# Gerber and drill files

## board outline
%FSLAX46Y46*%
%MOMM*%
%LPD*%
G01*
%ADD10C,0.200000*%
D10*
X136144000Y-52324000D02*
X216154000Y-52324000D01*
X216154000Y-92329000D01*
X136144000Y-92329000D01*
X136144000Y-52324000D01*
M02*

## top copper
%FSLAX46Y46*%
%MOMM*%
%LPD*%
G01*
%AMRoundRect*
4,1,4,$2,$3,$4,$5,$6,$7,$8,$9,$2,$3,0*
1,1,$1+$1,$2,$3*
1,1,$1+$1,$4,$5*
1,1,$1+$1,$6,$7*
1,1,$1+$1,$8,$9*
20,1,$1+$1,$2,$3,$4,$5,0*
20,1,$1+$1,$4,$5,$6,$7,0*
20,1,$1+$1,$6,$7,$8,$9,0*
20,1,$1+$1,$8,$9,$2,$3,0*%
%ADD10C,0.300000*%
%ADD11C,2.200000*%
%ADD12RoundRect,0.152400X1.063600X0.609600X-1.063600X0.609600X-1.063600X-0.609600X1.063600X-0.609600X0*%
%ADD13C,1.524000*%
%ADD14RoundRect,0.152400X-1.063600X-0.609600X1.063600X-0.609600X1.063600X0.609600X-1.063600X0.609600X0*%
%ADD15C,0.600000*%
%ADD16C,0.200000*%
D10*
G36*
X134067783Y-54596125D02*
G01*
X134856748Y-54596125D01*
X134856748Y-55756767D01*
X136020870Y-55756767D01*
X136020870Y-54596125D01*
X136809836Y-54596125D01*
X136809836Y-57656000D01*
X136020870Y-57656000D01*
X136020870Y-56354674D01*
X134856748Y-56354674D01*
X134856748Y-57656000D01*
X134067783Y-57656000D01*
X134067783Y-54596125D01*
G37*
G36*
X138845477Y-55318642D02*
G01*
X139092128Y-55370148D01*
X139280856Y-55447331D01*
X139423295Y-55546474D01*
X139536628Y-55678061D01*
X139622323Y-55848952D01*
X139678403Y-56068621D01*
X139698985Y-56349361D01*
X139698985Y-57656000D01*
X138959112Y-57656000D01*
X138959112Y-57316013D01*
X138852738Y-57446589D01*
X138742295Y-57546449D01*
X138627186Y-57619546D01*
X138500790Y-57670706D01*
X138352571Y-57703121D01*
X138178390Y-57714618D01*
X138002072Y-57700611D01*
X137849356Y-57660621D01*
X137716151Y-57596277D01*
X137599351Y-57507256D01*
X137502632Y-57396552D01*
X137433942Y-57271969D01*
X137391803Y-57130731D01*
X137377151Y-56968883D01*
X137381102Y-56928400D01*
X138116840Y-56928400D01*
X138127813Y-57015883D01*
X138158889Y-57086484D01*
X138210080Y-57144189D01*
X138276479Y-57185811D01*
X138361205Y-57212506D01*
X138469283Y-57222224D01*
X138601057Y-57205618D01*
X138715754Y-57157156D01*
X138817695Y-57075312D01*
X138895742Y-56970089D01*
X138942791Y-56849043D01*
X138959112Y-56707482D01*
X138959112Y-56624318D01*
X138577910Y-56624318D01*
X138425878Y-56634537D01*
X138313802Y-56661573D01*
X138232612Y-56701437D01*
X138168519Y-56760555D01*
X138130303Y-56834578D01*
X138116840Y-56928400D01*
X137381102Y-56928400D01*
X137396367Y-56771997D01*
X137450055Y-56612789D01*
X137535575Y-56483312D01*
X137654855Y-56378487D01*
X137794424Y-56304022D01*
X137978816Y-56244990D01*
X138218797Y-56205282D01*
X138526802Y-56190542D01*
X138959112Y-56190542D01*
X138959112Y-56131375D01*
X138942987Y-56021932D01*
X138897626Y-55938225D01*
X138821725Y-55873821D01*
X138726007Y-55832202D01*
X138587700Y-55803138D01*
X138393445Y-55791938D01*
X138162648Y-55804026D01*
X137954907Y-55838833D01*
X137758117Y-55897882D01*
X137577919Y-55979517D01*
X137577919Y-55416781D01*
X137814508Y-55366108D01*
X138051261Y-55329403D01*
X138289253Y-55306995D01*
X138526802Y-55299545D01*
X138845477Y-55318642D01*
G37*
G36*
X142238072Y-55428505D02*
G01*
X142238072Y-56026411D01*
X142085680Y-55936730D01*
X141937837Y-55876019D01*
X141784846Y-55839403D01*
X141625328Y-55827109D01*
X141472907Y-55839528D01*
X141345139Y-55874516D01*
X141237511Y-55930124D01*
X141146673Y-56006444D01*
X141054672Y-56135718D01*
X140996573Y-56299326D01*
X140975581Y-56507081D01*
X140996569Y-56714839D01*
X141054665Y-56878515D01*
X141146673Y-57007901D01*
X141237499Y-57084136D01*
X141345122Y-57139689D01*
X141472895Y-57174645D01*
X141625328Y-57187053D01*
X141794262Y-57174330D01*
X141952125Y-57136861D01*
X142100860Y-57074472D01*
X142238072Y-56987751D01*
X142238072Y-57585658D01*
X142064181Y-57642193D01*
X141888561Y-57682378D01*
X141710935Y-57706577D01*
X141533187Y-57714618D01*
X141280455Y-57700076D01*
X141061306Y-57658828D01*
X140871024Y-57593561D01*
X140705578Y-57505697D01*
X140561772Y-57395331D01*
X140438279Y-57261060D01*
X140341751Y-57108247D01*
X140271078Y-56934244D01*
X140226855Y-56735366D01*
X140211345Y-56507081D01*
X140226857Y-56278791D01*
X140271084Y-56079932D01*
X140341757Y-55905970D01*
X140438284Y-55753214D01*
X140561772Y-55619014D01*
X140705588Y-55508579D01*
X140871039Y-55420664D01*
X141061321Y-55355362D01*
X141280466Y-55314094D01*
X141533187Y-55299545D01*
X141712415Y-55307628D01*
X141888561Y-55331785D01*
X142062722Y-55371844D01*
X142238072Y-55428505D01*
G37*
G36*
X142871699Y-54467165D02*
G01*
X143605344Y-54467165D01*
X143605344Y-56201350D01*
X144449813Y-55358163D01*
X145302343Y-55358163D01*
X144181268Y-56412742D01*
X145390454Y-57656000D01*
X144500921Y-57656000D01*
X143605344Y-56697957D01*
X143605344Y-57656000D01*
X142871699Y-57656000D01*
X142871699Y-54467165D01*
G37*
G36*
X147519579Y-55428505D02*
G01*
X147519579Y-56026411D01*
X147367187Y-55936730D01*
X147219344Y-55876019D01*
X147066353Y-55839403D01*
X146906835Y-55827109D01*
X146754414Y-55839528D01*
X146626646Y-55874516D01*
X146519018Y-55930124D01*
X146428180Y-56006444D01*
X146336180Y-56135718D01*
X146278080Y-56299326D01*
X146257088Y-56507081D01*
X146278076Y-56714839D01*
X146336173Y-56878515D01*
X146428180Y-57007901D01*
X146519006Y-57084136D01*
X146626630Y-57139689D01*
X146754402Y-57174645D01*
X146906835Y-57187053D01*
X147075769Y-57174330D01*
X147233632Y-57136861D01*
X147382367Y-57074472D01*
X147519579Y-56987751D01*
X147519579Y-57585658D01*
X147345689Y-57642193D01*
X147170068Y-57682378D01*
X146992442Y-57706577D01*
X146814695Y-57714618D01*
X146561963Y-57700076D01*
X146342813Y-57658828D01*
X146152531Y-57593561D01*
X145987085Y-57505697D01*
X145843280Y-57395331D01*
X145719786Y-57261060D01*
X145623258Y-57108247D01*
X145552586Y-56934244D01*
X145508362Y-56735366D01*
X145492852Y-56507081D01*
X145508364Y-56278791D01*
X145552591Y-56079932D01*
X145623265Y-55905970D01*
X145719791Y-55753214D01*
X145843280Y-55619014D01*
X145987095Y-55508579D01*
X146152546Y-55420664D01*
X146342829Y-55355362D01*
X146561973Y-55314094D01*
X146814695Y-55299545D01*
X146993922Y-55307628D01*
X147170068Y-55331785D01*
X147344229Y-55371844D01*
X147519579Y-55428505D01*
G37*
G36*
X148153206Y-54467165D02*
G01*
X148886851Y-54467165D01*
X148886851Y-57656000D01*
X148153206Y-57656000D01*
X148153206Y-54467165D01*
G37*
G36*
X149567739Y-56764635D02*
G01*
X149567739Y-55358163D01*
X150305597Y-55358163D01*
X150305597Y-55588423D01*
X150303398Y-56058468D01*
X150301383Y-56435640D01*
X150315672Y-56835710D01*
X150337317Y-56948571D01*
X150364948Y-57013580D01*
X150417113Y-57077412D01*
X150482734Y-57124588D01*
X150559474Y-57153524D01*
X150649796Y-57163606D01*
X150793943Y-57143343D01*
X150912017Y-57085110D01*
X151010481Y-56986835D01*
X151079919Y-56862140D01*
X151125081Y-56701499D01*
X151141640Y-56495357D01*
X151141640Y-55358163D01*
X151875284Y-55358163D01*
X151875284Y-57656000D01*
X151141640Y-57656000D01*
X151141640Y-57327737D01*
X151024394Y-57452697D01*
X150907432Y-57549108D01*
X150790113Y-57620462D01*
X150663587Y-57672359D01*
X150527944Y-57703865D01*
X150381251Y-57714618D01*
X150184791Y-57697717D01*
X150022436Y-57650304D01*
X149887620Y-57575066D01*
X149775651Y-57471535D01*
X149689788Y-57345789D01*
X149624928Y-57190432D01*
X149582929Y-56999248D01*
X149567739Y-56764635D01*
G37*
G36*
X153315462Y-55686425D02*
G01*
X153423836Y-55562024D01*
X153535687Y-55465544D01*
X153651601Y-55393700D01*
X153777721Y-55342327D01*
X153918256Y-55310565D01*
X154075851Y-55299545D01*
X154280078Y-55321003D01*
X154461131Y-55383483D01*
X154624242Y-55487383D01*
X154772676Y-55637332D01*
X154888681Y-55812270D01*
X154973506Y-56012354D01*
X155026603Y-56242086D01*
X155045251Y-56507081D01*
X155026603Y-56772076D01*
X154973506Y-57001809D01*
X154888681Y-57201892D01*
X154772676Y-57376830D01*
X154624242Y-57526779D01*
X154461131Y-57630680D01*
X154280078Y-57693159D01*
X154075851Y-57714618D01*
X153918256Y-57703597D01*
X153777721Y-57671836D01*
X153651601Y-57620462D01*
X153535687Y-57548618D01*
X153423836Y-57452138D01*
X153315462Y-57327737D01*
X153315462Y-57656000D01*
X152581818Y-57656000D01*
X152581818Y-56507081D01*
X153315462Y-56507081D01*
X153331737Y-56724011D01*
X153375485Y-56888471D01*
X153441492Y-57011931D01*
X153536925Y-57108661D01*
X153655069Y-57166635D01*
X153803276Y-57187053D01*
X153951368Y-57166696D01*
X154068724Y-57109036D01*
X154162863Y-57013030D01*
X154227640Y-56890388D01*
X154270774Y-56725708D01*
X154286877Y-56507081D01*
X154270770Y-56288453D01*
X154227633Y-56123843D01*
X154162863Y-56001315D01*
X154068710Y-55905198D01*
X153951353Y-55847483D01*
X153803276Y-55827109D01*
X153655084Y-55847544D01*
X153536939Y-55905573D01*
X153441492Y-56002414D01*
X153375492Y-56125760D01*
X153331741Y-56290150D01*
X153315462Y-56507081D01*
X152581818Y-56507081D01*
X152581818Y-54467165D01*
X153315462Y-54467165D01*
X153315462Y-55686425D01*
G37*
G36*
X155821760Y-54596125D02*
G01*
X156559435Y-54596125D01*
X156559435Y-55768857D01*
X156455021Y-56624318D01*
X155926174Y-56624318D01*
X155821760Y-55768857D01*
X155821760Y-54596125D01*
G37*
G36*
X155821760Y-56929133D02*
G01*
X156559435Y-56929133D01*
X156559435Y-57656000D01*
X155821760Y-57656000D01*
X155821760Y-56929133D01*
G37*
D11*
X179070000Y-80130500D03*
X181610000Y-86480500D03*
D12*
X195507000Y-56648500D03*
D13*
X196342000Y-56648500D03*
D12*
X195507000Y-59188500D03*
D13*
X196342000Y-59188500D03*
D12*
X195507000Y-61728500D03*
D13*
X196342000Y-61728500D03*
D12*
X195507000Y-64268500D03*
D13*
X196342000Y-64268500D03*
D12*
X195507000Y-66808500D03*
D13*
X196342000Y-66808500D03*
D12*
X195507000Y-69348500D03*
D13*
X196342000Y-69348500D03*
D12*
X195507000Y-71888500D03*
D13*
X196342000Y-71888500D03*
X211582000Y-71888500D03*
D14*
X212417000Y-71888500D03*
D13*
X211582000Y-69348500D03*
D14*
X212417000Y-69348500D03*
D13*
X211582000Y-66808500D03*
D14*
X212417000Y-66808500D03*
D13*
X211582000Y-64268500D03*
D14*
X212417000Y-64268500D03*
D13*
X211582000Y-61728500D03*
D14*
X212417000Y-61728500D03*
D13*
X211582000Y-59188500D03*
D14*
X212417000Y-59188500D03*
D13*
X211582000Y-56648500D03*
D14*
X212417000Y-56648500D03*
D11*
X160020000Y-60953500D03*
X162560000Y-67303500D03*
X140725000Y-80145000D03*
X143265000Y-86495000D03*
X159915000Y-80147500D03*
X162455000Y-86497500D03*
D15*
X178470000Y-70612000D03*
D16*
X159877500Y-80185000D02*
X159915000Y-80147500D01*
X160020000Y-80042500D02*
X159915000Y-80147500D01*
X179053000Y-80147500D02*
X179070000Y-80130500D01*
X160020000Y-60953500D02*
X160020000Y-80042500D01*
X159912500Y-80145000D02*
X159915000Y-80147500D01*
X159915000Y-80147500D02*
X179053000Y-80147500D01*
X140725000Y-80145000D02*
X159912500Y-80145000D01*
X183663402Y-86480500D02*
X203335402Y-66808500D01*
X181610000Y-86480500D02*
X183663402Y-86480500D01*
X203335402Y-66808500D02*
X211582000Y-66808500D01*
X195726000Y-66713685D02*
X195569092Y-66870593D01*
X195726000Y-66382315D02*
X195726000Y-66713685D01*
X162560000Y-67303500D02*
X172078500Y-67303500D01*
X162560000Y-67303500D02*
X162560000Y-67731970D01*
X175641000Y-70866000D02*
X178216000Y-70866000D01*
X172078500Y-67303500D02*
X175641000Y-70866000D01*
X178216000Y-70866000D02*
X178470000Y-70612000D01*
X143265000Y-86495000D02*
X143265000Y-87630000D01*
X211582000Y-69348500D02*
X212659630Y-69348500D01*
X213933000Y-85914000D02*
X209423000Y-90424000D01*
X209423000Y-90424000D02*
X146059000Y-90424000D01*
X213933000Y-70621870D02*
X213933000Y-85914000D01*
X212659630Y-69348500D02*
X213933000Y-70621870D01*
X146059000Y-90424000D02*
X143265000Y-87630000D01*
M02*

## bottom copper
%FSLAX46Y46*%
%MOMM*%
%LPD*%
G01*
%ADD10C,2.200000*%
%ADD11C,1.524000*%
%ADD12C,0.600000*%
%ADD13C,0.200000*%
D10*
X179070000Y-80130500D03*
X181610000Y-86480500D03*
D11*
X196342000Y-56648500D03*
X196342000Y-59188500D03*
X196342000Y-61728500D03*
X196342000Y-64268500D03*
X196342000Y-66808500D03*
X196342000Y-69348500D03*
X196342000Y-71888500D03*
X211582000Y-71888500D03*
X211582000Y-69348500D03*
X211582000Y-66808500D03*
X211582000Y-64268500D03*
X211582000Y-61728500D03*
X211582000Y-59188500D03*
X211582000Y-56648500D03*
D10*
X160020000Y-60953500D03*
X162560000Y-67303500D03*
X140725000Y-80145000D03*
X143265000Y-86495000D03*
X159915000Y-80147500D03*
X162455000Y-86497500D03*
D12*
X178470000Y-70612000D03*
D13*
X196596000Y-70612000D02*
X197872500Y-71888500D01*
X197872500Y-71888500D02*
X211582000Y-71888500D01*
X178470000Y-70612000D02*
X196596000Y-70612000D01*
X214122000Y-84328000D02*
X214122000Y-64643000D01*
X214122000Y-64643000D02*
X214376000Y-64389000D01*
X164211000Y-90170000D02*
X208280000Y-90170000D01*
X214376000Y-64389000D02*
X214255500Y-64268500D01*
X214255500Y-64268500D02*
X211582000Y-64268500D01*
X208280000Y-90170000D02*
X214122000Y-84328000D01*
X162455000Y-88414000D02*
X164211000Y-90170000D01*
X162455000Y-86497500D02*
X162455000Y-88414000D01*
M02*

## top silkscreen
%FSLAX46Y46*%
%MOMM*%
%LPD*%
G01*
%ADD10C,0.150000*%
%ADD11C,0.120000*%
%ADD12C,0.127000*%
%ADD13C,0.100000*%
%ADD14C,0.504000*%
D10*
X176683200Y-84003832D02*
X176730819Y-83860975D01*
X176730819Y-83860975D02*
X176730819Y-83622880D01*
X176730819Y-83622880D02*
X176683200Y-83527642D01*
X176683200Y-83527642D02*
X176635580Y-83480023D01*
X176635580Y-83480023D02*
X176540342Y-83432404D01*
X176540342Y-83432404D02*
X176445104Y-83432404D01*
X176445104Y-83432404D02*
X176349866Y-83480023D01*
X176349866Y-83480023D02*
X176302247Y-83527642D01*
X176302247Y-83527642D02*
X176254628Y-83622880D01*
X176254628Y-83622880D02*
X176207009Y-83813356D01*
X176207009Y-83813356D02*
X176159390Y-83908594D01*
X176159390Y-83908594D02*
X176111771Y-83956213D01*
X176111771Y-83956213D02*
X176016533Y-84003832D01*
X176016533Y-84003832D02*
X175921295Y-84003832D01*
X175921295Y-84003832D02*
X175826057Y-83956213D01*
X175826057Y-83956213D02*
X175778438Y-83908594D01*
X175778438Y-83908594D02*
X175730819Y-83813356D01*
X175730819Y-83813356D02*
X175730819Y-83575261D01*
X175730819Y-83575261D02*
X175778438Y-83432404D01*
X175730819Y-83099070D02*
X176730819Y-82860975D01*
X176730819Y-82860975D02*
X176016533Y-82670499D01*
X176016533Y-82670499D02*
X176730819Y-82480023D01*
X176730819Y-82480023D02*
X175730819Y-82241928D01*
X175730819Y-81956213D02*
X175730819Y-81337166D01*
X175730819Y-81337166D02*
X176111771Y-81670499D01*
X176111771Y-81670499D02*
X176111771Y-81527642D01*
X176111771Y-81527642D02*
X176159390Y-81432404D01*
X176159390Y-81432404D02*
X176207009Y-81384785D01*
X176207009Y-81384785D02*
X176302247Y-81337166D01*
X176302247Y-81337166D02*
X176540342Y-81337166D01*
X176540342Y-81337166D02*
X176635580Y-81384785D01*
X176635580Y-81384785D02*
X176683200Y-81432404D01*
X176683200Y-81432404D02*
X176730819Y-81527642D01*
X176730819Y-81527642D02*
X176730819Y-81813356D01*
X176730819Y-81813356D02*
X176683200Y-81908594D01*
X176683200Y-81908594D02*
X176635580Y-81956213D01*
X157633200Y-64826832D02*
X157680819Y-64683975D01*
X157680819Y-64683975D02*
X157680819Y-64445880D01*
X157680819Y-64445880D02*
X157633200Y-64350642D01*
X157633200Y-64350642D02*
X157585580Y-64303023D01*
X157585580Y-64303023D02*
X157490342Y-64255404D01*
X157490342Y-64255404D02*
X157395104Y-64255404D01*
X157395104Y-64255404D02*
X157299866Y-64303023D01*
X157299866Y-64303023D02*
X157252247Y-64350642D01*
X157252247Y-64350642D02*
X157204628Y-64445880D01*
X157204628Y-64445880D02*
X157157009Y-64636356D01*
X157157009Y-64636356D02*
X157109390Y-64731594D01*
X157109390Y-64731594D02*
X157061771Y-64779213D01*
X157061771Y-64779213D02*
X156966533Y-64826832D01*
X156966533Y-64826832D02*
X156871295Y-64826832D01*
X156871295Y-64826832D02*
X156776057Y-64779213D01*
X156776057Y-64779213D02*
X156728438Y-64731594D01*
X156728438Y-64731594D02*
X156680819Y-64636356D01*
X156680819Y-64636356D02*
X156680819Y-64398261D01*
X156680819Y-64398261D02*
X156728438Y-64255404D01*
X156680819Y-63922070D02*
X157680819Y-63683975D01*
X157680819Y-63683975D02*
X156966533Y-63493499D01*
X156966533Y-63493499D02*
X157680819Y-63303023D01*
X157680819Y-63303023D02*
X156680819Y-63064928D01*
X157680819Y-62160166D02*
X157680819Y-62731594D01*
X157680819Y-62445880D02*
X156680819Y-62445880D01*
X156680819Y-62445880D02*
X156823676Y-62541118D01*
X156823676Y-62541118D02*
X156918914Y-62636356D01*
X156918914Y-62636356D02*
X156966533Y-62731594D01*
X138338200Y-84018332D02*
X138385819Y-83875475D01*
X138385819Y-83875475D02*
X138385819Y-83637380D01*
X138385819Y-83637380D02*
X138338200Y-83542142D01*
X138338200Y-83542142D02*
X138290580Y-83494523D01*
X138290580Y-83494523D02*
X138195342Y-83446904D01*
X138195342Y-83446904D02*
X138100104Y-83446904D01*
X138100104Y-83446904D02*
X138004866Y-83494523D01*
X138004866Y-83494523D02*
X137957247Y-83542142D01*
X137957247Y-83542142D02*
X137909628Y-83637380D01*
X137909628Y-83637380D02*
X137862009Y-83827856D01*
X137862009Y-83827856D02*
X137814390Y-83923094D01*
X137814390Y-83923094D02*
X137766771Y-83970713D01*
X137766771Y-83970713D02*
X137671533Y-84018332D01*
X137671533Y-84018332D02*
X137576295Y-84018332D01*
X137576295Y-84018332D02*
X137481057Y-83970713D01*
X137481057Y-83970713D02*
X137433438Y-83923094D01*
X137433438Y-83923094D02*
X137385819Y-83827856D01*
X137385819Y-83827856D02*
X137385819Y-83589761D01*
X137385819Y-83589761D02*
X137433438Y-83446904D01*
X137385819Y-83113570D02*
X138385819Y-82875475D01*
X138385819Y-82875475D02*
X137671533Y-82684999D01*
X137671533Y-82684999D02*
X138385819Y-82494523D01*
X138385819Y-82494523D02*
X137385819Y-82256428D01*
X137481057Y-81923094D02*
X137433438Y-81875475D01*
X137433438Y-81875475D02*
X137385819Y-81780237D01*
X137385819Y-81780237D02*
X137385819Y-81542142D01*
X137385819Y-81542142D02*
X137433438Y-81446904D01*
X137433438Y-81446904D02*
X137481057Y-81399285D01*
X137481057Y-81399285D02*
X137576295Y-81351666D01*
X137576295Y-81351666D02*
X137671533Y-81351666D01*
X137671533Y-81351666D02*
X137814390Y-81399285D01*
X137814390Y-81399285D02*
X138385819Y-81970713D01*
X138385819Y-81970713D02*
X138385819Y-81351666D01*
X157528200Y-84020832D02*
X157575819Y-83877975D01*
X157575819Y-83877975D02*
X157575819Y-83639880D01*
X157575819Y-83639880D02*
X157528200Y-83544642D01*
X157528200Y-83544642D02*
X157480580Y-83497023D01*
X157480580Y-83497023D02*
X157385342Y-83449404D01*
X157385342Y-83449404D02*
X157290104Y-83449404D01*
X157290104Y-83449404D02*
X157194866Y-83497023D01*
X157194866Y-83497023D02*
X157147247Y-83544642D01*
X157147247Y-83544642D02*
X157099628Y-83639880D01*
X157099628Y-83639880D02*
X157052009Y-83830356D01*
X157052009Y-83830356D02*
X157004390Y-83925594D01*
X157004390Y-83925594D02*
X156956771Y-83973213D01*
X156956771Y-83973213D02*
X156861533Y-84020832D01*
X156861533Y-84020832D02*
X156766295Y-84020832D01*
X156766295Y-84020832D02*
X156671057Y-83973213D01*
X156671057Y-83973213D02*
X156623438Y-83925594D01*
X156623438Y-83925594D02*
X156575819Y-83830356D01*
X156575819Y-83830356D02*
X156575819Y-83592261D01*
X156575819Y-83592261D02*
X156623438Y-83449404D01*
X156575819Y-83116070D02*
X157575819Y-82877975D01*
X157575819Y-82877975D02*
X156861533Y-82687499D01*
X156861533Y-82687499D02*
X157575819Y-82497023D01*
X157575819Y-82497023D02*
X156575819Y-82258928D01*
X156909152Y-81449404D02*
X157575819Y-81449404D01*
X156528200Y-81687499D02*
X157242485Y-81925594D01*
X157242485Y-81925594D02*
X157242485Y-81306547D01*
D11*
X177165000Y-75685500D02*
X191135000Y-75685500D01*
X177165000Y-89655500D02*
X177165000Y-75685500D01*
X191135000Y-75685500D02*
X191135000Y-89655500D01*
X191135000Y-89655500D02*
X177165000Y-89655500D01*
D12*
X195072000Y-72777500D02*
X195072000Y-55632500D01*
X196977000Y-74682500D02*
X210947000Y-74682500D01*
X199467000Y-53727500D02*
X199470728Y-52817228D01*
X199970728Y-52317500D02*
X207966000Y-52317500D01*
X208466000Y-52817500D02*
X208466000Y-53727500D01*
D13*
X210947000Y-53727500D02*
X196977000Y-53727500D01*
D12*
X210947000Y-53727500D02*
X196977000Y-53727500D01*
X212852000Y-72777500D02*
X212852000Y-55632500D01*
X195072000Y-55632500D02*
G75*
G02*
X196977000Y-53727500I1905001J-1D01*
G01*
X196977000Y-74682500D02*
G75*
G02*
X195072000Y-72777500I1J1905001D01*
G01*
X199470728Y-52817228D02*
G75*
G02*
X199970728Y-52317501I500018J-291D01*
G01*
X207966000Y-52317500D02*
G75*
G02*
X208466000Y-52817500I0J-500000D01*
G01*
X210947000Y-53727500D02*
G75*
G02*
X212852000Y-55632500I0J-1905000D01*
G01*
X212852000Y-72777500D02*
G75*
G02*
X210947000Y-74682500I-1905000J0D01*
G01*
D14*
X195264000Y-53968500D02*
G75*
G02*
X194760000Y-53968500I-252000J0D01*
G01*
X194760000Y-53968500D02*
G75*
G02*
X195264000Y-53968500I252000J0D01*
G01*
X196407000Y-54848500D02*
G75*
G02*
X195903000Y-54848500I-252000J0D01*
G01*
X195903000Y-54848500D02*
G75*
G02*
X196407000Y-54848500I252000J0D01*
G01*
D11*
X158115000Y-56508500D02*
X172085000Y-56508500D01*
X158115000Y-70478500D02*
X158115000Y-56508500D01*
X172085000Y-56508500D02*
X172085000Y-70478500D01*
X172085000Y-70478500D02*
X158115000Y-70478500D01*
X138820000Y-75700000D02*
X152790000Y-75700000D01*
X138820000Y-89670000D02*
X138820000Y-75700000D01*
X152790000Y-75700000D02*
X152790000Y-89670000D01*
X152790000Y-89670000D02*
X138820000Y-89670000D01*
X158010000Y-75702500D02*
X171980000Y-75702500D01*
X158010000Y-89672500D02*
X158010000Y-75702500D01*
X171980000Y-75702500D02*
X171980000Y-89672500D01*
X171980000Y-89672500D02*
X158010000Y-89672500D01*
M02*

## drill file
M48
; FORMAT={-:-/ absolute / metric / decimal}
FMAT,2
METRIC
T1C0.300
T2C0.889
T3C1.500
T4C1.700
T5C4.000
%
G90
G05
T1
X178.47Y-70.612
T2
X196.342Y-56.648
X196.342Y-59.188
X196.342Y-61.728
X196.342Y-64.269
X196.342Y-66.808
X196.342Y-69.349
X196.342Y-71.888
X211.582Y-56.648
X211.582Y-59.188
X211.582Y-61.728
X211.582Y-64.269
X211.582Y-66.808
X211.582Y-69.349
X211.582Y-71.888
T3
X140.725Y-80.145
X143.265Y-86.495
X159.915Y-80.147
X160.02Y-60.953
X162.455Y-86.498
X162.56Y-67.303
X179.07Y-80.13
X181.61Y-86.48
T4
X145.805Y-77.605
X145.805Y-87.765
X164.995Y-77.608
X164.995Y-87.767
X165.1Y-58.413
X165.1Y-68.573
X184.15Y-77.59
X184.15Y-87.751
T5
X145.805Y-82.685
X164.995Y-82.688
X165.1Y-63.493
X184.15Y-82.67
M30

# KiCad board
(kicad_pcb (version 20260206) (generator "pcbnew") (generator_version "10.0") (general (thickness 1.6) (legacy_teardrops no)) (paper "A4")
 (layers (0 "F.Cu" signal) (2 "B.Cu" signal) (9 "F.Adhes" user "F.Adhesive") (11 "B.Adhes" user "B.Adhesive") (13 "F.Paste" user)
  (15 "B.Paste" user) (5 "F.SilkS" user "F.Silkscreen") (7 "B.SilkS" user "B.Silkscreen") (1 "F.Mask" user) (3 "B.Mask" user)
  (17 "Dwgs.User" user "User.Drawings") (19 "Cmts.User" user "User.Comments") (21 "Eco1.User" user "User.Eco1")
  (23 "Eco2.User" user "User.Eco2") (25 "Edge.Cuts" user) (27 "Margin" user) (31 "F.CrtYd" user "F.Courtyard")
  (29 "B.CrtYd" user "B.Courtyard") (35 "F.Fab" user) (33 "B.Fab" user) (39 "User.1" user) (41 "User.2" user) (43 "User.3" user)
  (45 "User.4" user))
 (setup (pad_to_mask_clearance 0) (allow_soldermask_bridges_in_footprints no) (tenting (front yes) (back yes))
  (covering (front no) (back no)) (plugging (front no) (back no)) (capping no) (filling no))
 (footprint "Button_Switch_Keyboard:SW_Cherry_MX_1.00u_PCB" (layer "F.Cu") (at 179.07 80.1305 90)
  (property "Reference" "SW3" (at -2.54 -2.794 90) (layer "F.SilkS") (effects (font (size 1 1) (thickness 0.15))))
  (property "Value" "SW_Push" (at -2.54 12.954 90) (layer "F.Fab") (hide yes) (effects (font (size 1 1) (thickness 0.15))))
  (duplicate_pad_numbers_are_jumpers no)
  (fp_line (start 4.445 -1.905) (end 4.445 12.065) (stroke (width 0.12) (type solid)) (layer "F.SilkS"))
  (fp_line (start -9.525 -1.905) (end 4.445 -1.905) (stroke (width 0.12) (type solid)) (layer "F.SilkS"))
  (fp_line (start 4.445 12.065) (end -9.525 12.065) (stroke (width 0.12) (type solid)) (layer "F.SilkS"))
  (fp_line (start -9.525 12.065) (end -9.525 -1.905) (stroke (width 0.12) (type solid)) (layer "F.SilkS"))
  (pad "" np_thru_hole circle (at -7.62 5.08 90) (size 1.7 1.7) (drill 1.7) (layers "*.Cu" "*.Mask"))
  (pad "" np_thru_hole circle (at -2.54 5.08 90) (size 4 4) (drill 4) (layers "*.Cu" "*.Mask"))
  (pad "" np_thru_hole circle (at 2.54 5.08 90) (size 1.7 1.7) (drill 1.7) (layers "*.Cu" "*.Mask"))
  (pad "1" thru_hole circle (at 0 0 90) (size 2.2 2.2) (drill 1.5) (layers "*.Cu" "*.Mask") (remove_unused_layers no) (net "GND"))
  (pad "2" thru_hole circle (at -6.35 2.54 90) (size 2.2 2.2) (drill 1.5) (layers "*.Cu" "*.Mask") (remove_unused_layers no)
   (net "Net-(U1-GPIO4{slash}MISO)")))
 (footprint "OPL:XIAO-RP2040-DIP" (layer "F.Cu") (at 203.962 64.2685)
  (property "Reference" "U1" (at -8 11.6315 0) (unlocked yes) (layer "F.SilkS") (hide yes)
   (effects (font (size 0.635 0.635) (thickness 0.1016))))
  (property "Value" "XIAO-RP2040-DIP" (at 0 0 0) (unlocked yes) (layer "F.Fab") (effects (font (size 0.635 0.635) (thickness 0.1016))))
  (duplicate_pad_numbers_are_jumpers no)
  (fp_line (start -8.89 8.509) (end -8.89 -8.636) (stroke (width 0.127) (type solid)) (layer "F.SilkS"))
  (fp_line (start -6.985 10.414) (end 6.985 10.414) (stroke (width 0.127) (type solid)) (layer "F.SilkS"))
  (fp_line (start -4.495 -10.541) (end -4.491272 -11.451272) (stroke (width 0.127) (type solid)) (layer "F.SilkS"))
  (fp_line (start -3.991272 -11.951) (end 4.004 -11.951) (stroke (width 0.127) (type solid)) (layer "F.SilkS"))
  (fp_line (start 4.504 -11.451) (end 4.504 -10.541) (stroke (width 0.127) (type solid)) (layer "F.SilkS"))
  (fp_line (start 6.985 -10.541) (end -6.985 -10.541) (stroke (width 0.1) (type solid)) (layer "F.SilkS"))
  (fp_line (start 6.985 -10.541) (end -6.985 -10.541) (stroke (width 0.127) (type solid)) (layer "F.SilkS"))
  (fp_line (start 8.89 8.509) (end 8.89 -8.636) (stroke (width 0.127) (type solid)) (layer "F.SilkS"))
  (fp_arc (start -8.89 -8.636) (mid -8.332038 -9.983038) (end -6.985 -10.541) (stroke (width 0.127) (type solid)) (layer "F.SilkS"))
  (fp_arc (start -6.985 10.414) (mid -8.332038 9.856038) (end -8.89 8.509) (stroke (width 0.127) (type solid)) (layer "F.SilkS"))
  (fp_arc (start -4.491272 -11.451272) (mid -4.344728 -11.80464) (end -3.991272 -11.951) (stroke (width 0.127) (type default))
   (layer "F.SilkS"))
  (fp_arc (start 4.004 -11.951) (mid 4.357553 -11.804553) (end 4.504 -11.451) (stroke (width 0.127) (type default)) (layer "F.SilkS"))
  (fp_arc (start 6.985 -10.541) (mid 8.332038 -9.983038) (end 8.89 -8.636) (stroke (width 0.127) (type solid)) (layer "F.SilkS"))
  (fp_arc (start 8.89 8.509) (mid 8.332038 9.856038) (end 6.985 10.414) (stroke (width 0.127) (type solid)) (layer "F.SilkS"))
  (fp_circle (center -8.95 -10.3) (end -8.95 -10.554) (stroke (width 0.5) (type solid)) (fill yes) (layer "F.SilkS"))
  (fp_circle (center -7.807 -9.42) (end -7.807 -9.674) (stroke (width 0.5) (type solid)) (fill yes) (layer "F.SilkS"))
  (pad "1" smd roundrect (at -8.455 -7.62 180) (size 2.432 1.524) (layers "F.Cu" "F.Mask") (roundrect_rratio 0.1)
   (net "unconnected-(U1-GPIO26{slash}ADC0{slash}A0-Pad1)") (thermal_bridge_angle 45))
  (pad "1" thru_hole circle (at -7.62 -7.62 180) (size 1.524 1.524) (drill 0.889) (layers "*.Cu" "*.Mask") (remove_unused_layers no)
   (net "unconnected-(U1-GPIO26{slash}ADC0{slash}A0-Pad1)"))
  (pad "2" smd roundrect (at -8.455 -5.08 180) (size 2.432 1.524) (layers "F.Cu" "F.Mask") (roundrect_rratio 0.1)
   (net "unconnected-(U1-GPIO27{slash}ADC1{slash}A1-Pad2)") (thermal_bridge_angle 45))
  (pad "2" thru_hole circle (at -7.62 -5.08 180) (size 1.524 1.524) (drill 0.889) (layers "*.Cu" "*.Mask") (remove_unused_layers no)
   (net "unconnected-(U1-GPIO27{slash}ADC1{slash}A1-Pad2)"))
  (pad "3" smd roundrect (at -8.455 -2.54 180) (size 2.432 1.524) (layers "F.Cu" "F.Mask") (roundrect_rratio 0.1)
   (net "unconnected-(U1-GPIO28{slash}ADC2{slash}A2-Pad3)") (thermal_bridge_angle 45))
  (pad "3" thru_hole circle (at -7.62 -2.54 180) (size 1.524 1.524) (drill 0.889) (layers "*.Cu" "*.Mask") (remove_unused_layers no)
   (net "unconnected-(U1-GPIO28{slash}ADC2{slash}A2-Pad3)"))
  (pad "4" smd roundrect (at -8.455 0 180) (size 2.432 1.524) (layers "F.Cu" "F.Mask") (roundrect_rratio 0.1)
   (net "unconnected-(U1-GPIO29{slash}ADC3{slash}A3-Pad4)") (thermal_bridge_angle 45))
  (pad "4" thru_hole circle (at -7.62 0 180) (size 1.524 1.524) (drill 0.889) (layers "*.Cu" "*.Mask") (remove_unused_layers no)
   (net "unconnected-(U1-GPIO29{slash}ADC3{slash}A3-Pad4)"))
  (pad "5" smd roundrect (at -8.455 2.54 180) (size 2.432 1.524) (layers "F.Cu" "F.Mask") (roundrect_rratio 0.1) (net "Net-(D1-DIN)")
   (thermal_bridge_angle 45))
  (pad "5" thru_hole circle (at -7.62 2.54 180) (size 1.524 1.524) (drill 0.889) (layers "*.Cu" "*.Mask") (remove_unused_layers no)
   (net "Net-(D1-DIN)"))
  (pad "6" smd roundrect (at -8.455 5.08 180) (size 2.432 1.524) (layers "F.Cu" "F.Mask") (roundrect_rratio 0.1)
   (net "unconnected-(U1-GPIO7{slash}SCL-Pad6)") (thermal_bridge_angle 45))
  (pad "6" thru_hole circle (at -7.62 5.08 180) (size 1.524 1.524) (drill 0.889) (layers "*.Cu" "*.Mask") (remove_unused_layers no)
   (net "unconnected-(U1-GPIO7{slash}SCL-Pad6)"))
  (pad "7" smd roundrect (at -8.455 7.62 180) (size 2.432 1.524) (layers "F.Cu" "F.Mask") (roundrect_rratio 0.1)
   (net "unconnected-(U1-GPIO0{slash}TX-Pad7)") (thermal_bridge_angle 45))
  (pad "7" thru_hole circle (at -7.62 7.62 180) (size 1.524 1.524) (drill 0.889) (layers "*.Cu" "*.Mask") (remove_unused_layers no)
   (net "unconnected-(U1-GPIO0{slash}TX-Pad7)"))
  (pad "8" thru_hole circle (at 7.62 7.62) (size 1.524 1.524) (drill 0.889) (layers "*.Cu" "*.Mask") (remove_unused_layers no)
   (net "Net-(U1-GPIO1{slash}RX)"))
  (pad "8" smd roundrect (at 8.455 7.62) (size 2.432 1.524) (layers "F.Cu" "F.Mask") (roundrect_rratio 0.1) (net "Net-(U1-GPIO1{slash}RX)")
   (thermal_bridge_angle 45))
  (pad "9" thru_hole circle (at 7.62 5.08) (size 1.524 1.524) (drill 0.889) (layers "*.Cu" "*.Mask") (remove_unused_layers no)
   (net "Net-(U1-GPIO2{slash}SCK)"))
  (pad "9" smd roundrect (at 8.455 5.08) (size 2.432 1.524) (layers "F.Cu" "F.Mask") (roundrect_rratio 0.1) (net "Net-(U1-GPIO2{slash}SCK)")
   (thermal_bridge_angle 45))
  (pad "10" thru_hole circle (at 7.62 2.54) (size 1.524 1.524) (drill 0.889) (layers "*.Cu" "*.Mask") (remove_unused_layers no)
   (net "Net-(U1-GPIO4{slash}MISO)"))
  (pad "10" smd roundrect (at 8.455 2.54) (size 2.432 1.524) (layers "F.Cu" "F.Mask") (roundrect_rratio 0.1)
   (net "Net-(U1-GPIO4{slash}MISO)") (thermal_bridge_angle 45))
  (pad "11" thru_hole circle (at 7.62 0) (size 1.524 1.524) (drill 0.889) (layers "*.Cu" "*.Mask") (remove_unused_layers no)
   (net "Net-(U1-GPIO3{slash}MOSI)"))
  (pad "11" smd roundrect (at 8.455 0) (size 2.432 1.524) (layers "F.Cu" "F.Mask") (roundrect_rratio 0.1) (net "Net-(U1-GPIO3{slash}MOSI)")
   (thermal_bridge_angle 45))
  (pad "12" thru_hole circle (at 7.62 -2.54) (size 1.524 1.524) (drill 0.889) (layers "*.Cu" "*.Mask") (remove_unused_layers no)
   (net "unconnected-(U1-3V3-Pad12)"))
  (pad "12" smd roundrect (at 8.455 -2.54) (size 2.432 1.524) (layers "F.Cu" "F.Mask") (roundrect_rratio 0.1)
   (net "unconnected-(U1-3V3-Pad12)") (thermal_bridge_angle 45))
  (pad "13" thru_hole circle (at 7.62 -5.08) (size 1.524 1.524) (drill 0.889) (layers "*.Cu" "*.Mask") (remove_unused_layers no)
   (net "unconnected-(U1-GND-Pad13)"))
  (pad "13" smd roundrect (at 8.455 -5.08) (size 2.432 1.524) (layers "F.Cu" "F.Mask") (roundrect_rratio 0.1)
   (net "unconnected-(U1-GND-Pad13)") (thermal_bridge_angle 45))
  (pad "14" thru_hole circle (at 7.62 -7.62) (size 1.524 1.524) (drill 0.889) (layers "*.Cu" "*.Mask") (remove_unused_layers no)
   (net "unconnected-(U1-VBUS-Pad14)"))
  (pad "14" smd roundrect (at 8.455 -7.62) (size 2.432 1.524) (layers "F.Cu" "F.Mask") (roundrect_rratio 0.1)
   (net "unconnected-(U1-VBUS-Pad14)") (thermal_bridge_angle 45)))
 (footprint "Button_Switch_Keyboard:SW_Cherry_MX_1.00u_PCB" (layer "F.Cu") (at 160.02 60.9535 90)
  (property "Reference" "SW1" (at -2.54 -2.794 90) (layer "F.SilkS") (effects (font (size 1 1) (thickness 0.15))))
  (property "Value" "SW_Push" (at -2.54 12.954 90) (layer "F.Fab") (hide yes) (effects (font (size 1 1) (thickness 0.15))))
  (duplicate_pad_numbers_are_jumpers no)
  (fp_line (start 4.445 -1.905) (end 4.445 12.065) (stroke (width 0.12) (type solid)) (layer "F.SilkS"))
  (fp_line (start -9.525 -1.905) (end 4.445 -1.905) (stroke (width 0.12) (type solid)) (layer "F.SilkS"))
  (fp_line (start 4.445 12.065) (end -9.525 12.065) (stroke (width 0.12) (type solid)) (layer "F.SilkS"))
  (fp_line (start -9.525 12.065) (end -9.525 -1.905) (stroke (width 0.12) (type solid)) (layer "F.SilkS"))
  (pad "" np_thru_hole circle (at -7.62 5.08 90) (size 1.7 1.7) (drill 1.7) (layers "*.Cu" "*.Mask"))
  (pad "" np_thru_hole circle (at -2.54 5.08 90) (size 4 4) (drill 4) (layers "*.Cu" "*.Mask"))
  (pad "" np_thru_hole circle (at 2.54 5.08 90) (size 1.7 1.7) (drill 1.7) (layers "*.Cu" "*.Mask"))
  (pad "1" thru_hole circle (at 0 0 90) (size 2.2 2.2) (drill 1.5) (layers "*.Cu" "*.Mask") (remove_unused_layers no) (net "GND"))
  (pad "2" thru_hole circle (at -6.35 2.54 90) (size 2.2 2.2) (drill 1.5) (layers "*.Cu" "*.Mask") (remove_unused_layers no)
   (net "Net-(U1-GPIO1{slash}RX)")))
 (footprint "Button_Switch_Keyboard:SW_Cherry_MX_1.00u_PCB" (layer "F.Cu") (at 140.725 80.145 90)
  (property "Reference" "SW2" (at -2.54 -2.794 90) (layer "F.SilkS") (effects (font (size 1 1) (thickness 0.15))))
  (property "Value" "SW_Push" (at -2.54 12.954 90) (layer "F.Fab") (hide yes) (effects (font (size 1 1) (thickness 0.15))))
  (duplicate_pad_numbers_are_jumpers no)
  (fp_line (start 4.445 -1.905) (end 4.445 12.065) (stroke (width 0.12) (type solid)) (layer "F.SilkS"))
  (fp_line (start -9.525 -1.905) (end 4.445 -1.905) (stroke (width 0.12) (type solid)) (layer "F.SilkS"))
  (fp_line (start 4.445 12.065) (end -9.525 12.065) (stroke (width 0.12) (type solid)) (layer "F.SilkS"))
  (fp_line (start -9.525 12.065) (end -9.525 -1.905) (stroke (width 0.12) (type solid)) (layer "F.SilkS"))
  (pad "" np_thru_hole circle (at -7.62 5.08 90) (size 1.7 1.7) (drill 1.7) (layers "*.Cu" "*.Mask"))
  (pad "" np_thru_hole circle (at -2.54 5.08 90) (size 4 4) (drill 4) (layers "*.Cu" "*.Mask"))
  (pad "" np_thru_hole circle (at 2.54 5.08 90) (size 1.7 1.7) (drill 1.7) (layers "*.Cu" "*.Mask"))
  (pad "1" thru_hole circle (at 0 0 90) (size 2.2 2.2) (drill 1.5) (layers "*.Cu" "*.Mask") (remove_unused_layers no) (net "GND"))
  (pad "2" thru_hole circle (at -6.35 2.54 90) (size 2.2 2.2) (drill 1.5) (layers "*.Cu" "*.Mask") (remove_unused_layers no)
   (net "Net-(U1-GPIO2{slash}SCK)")))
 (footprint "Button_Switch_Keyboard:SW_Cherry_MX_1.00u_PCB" (layer "F.Cu") (at 159.915 80.1475 90)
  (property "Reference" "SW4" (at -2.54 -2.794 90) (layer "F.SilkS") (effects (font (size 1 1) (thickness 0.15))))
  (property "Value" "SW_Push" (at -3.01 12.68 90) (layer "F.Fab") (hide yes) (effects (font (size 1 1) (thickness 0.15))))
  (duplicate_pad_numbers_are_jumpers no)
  (fp_line (start 4.445 -1.905) (end 4.445 12.065) (stroke (width 0.12) (type solid)) (layer "F.SilkS"))
  (fp_line (start -9.525 -1.905) (end 4.445 -1.905) (stroke (width 0.12) (type solid)) (layer "F.SilkS"))
  (fp_line (start 4.445 12.065) (end -9.525 12.065) (stroke (width 0.12) (type solid)) (layer "F.SilkS"))
  (fp_line (start -9.525 12.065) (end -9.525 -1.905) (stroke (width 0.12) (type solid)) (layer "F.SilkS"))
  (pad "" np_thru_hole circle (at -7.62 5.08 90) (size 1.7 1.7) (drill 1.7) (layers "*.Cu" "*.Mask"))
  (pad "" np_thru_hole circle (at -2.54 5.08 90) (size 4 4) (drill 4) (layers "*.Cu" "*.Mask"))
  (pad "" np_thru_hole circle (at 2.54 5.08 90) (size 1.7 1.7) (drill 1.7) (layers "*.Cu" "*.Mask"))
  (pad "1" thru_hole circle (at 0 0 90) (size 2.2 2.2) (drill 1.5) (layers "*.Cu" "*.Mask") (remove_unused_layers no) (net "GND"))
  (pad "2" thru_hole circle (at -6.35 2.54 90) (size 2.2 2.2) (drill 1.5) (layers "*.Cu" "*.Mask") (remove_unused_layers no)
   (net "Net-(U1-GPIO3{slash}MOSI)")))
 (gr_rect (start 136.144 52.324) (end 216.154 92.329) (stroke (width 0.2) (type default)) (fill no) (layer "Edge.Cuts"))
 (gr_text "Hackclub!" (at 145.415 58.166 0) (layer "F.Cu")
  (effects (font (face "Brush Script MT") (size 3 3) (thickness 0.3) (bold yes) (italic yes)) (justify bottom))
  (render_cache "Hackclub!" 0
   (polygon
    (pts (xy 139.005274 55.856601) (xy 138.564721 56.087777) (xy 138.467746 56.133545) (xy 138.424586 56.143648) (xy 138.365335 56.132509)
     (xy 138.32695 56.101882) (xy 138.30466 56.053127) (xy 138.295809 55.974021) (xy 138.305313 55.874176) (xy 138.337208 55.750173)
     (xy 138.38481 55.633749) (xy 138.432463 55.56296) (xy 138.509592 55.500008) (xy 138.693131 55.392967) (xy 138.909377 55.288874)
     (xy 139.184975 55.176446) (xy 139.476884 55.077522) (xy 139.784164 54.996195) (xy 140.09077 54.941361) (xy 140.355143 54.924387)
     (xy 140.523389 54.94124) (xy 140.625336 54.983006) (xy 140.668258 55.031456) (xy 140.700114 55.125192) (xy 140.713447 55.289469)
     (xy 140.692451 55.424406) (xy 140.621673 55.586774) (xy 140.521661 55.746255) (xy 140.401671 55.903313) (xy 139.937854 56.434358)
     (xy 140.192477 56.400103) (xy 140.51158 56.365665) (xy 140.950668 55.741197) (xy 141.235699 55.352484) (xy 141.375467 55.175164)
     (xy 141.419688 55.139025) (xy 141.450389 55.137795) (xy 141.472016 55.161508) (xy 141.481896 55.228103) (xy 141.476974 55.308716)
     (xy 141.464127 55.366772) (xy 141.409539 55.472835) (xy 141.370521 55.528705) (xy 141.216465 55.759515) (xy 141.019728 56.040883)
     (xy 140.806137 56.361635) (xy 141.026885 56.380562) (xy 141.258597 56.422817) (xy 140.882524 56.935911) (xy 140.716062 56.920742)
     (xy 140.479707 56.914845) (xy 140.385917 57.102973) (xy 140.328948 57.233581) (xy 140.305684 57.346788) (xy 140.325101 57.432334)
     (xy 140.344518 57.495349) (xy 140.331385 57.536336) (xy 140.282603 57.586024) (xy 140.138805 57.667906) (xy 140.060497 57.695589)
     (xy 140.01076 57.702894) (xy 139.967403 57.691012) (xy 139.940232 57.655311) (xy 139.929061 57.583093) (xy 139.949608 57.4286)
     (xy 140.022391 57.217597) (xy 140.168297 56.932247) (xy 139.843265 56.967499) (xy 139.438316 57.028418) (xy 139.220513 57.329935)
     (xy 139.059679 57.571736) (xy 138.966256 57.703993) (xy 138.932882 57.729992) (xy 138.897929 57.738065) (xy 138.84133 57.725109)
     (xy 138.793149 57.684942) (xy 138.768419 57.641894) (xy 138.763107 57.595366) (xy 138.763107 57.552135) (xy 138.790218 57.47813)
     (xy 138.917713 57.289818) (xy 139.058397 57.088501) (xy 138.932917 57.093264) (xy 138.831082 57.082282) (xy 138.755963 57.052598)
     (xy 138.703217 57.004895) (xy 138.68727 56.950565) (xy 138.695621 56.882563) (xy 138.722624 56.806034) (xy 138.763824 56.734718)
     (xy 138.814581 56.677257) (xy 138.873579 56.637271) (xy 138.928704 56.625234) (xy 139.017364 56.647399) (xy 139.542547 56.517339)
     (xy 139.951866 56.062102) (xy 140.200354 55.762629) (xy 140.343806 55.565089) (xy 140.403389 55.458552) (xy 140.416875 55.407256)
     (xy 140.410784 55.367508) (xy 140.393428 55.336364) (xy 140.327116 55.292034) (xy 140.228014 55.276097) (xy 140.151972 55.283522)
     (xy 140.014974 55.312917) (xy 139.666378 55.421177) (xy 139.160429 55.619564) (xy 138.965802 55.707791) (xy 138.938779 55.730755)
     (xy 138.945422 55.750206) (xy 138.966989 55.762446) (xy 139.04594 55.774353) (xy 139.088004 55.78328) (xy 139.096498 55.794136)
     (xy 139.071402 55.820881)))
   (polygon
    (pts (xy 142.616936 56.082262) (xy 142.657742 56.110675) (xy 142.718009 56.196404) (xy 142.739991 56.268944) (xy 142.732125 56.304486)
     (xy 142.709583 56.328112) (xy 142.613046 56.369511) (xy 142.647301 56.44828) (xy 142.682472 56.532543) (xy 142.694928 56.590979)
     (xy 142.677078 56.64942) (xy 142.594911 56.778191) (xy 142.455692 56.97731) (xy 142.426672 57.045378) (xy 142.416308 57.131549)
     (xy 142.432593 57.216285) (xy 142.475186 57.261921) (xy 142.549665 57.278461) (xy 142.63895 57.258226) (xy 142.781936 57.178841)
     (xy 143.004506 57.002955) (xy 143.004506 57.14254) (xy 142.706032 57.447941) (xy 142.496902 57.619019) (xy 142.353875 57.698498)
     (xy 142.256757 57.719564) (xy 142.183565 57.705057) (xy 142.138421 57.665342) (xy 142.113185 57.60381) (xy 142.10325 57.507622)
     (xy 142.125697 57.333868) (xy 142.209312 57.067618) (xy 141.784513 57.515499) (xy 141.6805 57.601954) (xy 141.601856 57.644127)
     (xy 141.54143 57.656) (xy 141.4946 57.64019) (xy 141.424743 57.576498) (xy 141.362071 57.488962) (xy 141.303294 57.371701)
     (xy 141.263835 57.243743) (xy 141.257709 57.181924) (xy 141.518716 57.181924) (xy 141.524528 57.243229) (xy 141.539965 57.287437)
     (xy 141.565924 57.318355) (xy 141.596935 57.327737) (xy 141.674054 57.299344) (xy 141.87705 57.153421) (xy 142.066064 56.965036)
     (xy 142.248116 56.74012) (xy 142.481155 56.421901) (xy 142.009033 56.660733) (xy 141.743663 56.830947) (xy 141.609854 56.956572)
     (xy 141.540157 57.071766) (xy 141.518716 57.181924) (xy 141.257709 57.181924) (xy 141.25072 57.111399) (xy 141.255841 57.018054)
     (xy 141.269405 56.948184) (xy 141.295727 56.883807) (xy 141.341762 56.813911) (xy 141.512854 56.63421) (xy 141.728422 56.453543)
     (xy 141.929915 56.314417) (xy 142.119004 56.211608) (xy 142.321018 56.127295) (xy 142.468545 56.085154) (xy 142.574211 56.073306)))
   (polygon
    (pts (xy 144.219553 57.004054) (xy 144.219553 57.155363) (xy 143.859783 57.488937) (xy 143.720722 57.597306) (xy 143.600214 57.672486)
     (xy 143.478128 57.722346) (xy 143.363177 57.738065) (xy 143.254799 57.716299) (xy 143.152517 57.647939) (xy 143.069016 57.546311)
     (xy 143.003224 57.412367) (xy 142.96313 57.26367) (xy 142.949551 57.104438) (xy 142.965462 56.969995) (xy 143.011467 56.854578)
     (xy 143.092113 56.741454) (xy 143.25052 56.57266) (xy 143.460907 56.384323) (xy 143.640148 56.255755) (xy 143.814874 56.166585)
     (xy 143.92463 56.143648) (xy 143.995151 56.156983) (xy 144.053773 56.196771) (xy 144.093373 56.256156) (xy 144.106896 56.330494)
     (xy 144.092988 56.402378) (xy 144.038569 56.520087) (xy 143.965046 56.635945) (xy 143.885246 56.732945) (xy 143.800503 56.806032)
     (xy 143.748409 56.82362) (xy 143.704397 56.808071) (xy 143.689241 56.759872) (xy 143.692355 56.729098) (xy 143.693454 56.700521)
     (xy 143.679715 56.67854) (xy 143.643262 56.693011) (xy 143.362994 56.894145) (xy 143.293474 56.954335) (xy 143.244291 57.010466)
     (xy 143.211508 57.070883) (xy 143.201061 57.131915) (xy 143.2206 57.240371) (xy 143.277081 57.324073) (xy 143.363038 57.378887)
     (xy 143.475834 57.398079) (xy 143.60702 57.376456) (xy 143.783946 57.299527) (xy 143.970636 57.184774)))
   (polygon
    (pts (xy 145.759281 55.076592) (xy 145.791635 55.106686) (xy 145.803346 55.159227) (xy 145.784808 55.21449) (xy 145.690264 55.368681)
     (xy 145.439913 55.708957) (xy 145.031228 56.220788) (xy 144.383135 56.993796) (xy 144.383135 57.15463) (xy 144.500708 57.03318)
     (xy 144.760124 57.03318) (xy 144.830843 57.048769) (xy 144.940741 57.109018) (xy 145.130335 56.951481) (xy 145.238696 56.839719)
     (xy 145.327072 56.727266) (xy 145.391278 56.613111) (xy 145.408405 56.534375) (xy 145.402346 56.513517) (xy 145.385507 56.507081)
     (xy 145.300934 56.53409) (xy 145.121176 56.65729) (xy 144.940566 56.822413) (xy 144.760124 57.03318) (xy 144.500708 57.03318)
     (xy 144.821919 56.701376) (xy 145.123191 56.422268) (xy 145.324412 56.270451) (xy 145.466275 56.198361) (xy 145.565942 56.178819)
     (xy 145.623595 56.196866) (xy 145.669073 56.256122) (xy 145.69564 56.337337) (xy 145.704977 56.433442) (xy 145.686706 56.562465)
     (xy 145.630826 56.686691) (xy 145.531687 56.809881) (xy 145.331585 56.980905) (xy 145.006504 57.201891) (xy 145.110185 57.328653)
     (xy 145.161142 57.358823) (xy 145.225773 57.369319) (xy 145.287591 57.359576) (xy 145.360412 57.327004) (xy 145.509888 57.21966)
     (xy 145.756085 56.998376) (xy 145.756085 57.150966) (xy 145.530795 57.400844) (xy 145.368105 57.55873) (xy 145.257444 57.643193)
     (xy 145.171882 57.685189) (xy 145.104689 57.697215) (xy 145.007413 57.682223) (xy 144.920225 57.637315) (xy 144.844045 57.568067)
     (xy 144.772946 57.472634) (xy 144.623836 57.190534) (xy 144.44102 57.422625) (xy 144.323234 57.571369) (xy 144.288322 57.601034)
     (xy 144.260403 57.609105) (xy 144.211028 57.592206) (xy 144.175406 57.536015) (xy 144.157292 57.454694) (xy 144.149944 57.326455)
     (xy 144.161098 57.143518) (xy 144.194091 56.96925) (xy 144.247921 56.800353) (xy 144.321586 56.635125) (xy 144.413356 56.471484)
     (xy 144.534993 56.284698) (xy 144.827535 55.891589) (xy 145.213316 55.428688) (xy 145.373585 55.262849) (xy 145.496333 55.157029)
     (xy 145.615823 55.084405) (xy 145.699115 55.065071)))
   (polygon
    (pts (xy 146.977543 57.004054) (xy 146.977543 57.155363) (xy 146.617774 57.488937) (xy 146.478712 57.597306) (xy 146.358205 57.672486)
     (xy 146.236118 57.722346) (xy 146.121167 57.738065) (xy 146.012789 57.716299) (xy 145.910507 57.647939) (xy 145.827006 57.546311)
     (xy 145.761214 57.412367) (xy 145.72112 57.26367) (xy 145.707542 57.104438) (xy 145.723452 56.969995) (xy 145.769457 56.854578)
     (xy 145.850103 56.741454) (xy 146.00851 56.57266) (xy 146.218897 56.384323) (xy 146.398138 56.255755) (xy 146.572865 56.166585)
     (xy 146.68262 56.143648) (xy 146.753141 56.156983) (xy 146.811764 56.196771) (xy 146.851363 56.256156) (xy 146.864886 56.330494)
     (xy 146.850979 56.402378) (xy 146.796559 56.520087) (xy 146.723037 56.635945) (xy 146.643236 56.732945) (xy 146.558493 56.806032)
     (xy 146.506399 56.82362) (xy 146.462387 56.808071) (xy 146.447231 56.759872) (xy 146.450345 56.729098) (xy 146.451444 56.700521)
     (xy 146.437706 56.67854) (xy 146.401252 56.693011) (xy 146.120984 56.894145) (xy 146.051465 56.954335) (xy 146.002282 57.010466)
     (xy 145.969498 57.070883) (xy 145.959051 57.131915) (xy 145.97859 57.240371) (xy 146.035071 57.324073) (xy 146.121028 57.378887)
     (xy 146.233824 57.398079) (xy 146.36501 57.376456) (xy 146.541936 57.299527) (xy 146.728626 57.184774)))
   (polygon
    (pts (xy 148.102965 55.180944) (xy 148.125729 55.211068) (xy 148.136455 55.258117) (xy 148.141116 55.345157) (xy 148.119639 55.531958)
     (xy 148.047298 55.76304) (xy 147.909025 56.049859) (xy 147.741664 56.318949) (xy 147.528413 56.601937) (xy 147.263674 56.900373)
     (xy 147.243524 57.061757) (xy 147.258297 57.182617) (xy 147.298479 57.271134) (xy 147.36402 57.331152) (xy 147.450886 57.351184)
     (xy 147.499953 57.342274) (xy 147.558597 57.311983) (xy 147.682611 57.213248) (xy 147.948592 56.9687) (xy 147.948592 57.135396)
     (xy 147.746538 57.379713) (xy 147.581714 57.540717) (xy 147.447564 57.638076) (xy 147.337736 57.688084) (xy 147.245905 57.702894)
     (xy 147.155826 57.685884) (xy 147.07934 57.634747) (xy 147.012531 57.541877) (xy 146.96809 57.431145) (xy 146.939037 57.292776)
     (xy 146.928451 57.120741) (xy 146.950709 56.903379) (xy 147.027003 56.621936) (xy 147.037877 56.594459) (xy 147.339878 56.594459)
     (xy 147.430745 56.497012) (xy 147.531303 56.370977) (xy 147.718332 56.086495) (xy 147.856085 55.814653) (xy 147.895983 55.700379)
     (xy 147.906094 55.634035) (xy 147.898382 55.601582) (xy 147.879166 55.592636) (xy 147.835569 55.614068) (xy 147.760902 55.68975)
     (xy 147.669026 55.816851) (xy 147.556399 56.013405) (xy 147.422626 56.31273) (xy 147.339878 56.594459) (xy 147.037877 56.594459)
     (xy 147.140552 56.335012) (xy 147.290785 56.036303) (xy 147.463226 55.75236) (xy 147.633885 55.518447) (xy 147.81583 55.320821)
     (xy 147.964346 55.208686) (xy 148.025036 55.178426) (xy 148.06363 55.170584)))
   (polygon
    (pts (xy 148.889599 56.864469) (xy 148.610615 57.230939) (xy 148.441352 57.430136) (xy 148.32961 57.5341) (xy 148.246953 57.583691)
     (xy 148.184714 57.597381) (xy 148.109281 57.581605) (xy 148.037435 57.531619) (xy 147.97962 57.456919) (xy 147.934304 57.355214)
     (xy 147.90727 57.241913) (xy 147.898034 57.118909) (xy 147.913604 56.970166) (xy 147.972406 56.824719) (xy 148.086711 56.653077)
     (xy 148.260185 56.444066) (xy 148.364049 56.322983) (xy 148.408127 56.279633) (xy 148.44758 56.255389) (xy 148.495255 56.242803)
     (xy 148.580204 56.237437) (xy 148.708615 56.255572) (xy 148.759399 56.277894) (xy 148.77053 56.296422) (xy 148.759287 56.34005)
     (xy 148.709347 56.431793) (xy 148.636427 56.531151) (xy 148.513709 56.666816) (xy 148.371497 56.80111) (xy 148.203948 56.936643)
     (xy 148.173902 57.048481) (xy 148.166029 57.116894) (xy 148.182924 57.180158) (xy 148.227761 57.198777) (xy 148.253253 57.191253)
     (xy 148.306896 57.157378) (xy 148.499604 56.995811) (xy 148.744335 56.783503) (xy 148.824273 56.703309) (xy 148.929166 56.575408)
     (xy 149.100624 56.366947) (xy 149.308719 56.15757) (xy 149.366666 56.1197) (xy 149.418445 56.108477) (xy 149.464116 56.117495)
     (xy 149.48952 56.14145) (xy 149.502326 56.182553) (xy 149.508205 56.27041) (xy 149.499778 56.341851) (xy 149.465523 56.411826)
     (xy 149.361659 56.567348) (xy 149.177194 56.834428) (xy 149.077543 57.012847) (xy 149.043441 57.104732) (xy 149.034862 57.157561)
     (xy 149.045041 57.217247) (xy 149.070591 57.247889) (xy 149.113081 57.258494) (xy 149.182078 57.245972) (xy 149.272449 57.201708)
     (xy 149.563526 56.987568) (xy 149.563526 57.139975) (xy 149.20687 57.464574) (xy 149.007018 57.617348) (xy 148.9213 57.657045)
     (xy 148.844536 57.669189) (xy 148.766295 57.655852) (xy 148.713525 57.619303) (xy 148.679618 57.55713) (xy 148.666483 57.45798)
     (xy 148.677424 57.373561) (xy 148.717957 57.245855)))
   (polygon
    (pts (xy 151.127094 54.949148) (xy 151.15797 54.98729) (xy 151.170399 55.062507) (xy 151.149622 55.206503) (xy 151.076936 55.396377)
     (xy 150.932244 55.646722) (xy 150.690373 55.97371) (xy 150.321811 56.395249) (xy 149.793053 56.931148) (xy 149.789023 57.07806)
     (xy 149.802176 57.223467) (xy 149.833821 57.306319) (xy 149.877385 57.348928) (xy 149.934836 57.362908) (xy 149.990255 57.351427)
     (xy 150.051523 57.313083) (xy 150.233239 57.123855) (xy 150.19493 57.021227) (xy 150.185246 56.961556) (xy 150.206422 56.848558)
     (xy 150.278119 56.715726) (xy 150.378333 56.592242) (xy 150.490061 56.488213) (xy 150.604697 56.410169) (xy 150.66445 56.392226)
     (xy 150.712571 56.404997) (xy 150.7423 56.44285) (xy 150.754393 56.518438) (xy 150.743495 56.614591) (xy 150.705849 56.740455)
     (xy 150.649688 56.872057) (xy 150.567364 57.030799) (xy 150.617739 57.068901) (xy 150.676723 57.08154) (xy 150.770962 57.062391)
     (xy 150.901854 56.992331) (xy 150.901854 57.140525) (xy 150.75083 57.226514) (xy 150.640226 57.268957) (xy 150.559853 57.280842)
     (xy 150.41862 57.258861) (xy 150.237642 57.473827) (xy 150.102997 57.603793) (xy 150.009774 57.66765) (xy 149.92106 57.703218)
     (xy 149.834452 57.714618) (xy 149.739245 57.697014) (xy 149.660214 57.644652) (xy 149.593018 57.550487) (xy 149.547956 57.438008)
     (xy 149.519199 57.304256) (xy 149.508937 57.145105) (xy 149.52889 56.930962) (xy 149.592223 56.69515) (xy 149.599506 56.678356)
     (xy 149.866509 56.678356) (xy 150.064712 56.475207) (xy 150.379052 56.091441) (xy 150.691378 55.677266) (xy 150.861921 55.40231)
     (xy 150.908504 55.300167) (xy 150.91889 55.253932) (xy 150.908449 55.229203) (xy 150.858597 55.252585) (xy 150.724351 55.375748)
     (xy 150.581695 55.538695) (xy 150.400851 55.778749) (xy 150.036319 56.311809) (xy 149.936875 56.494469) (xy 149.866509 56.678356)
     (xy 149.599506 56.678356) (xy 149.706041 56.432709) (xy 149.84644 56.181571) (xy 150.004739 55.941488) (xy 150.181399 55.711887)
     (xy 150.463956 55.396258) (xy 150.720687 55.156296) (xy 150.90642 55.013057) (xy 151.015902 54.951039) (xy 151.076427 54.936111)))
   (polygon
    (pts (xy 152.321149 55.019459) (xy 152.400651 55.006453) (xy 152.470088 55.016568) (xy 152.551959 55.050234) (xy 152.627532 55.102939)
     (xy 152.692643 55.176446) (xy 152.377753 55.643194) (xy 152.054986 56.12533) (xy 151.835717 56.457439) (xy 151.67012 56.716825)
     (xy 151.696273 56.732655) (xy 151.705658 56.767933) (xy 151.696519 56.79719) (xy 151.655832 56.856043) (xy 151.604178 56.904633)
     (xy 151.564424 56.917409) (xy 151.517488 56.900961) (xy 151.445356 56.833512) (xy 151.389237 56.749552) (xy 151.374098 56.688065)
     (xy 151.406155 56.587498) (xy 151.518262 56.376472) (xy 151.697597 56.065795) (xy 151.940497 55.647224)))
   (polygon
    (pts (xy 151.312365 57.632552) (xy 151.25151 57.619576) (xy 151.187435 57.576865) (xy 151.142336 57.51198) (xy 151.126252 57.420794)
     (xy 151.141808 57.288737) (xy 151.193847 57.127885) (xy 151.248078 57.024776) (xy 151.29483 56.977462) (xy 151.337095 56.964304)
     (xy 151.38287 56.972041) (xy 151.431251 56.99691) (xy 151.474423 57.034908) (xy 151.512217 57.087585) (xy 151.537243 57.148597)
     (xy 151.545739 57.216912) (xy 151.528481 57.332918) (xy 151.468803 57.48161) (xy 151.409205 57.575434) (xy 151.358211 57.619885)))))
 (segment (start 159.8775 80.185) (end 159.915 80.1475) (width 0.2) (layer "F.Cu") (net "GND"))
 (segment (start 160.02 80.0425) (end 159.915 80.1475) (width 0.2) (layer "F.Cu") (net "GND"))
 (segment (start 179.053 80.1475) (end 179.07 80.1305) (width 0.2) (layer "F.Cu") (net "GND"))
 (segment (start 160.02 60.9535) (end 160.02 80.0425) (width 0.2) (layer "F.Cu") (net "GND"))
 (segment (start 159.9125 80.145) (end 159.915 80.1475) (width 0.2) (layer "F.Cu") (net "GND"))
 (segment (start 159.915 80.1475) (end 179.053 80.1475) (width 0.2) (layer "F.Cu") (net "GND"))
 (segment (start 140.725 80.145) (end 159.9125 80.145) (width 0.2) (layer "F.Cu") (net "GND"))
 (segment (start 183.663402 86.4805) (end 203.335402 66.8085) (width 0.2) (layer "F.Cu") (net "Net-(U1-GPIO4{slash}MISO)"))
 (segment (start 181.61 86.4805) (end 183.663402 86.4805) (width 0.2) (layer "F.Cu") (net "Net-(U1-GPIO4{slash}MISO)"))
 (segment (start 203.335402 66.8085) (end 211.582 66.8085) (width 0.2) (layer "F.Cu") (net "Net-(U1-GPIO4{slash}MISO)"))
 (segment (start 195.726 66.713685) (end 195.569092 66.870593) (width 0.2) (layer "F.Cu") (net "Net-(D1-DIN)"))
 (segment (start 195.726 66.382315) (end 195.726 66.713685) (width 0.2) (layer "F.Cu") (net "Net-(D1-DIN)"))
 (segment (start 162.56 67.3035) (end 172.0785 67.3035) (width 0.2) (layer "F.Cu") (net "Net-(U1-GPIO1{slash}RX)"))
 (segment (start 162.56 67.3035) (end 162.56 67.73197) (width 0.2) (layer "F.Cu") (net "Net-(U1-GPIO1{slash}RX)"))
 (segment (start 175.641 70.866) (end 178.216 70.866) (width 0.2) (layer "F.Cu") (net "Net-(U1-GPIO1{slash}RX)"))
 (segment (start 172.0785 67.3035) (end 175.641 70.866) (width 0.2) (layer "F.Cu") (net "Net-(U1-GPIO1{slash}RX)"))
 (segment (start 178.216 70.866) (end 178.47 70.612) (width 0.2) (layer "F.Cu") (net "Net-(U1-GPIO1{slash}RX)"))
 (via (at 178.47 70.612) (size 0.6) (drill 0.3) (layers "F.Cu" "B.Cu") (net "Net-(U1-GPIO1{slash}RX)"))
 (segment (start 196.596 70.612) (end 197.8725 71.8885) (width 0.2) (layer "B.Cu") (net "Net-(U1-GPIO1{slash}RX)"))
 (segment (start 197.8725 71.8885) (end 211.582 71.8885) (width 0.2) (layer "B.Cu") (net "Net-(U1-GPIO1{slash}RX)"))
 (segment (start 178.47 70.612) (end 196.596 70.612) (width 0.2) (layer "B.Cu") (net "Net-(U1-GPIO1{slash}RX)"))
 (segment (start 143.265 86.495) (end 143.265 87.63) (width 0.2) (layer "F.Cu") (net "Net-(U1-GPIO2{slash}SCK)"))
 (segment (start 211.582 69.3485) (end 212.65963 69.3485) (width 0.2) (layer "F.Cu") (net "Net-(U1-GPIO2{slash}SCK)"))
 (segment (start 213.933 85.914) (end 209.423 90.424) (width 0.2) (layer "F.Cu") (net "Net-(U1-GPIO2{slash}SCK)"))
 (segment (start 209.423 90.424) (end 146.059 90.424) (width 0.2) (layer "F.Cu") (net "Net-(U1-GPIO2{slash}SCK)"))
 (segment (start 213.933 70.62187) (end 213.933 85.914) (width 0.2) (layer "F.Cu") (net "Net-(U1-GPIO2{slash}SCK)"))
 (segment (start 212.65963 69.3485) (end 213.933 70.62187) (width 0.2) (layer "F.Cu") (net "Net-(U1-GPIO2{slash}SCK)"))
 (segment (start 146.059 90.424) (end 143.265 87.63) (width 0.2) (layer "F.Cu") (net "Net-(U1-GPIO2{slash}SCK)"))
 (segment (start 214.122 84.328) (end 214.122 64.643) (width 0.2) (layer "B.Cu") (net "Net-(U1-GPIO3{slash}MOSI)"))
 (segment (start 214.122 64.643) (end 214.376 64.389) (width 0.2) (layer "B.Cu") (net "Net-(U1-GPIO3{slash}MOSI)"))
 (segment (start 164.211 90.17) (end 208.28 90.17) (width 0.2) (layer "B.Cu") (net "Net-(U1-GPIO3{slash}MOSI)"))
 (segment (start 214.376 64.389) (end 214.2555 64.2685) (width 0.2) (layer "B.Cu") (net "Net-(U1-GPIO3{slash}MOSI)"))
 (segment (start 214.2555 64.2685) (end 211.582 64.2685) (width 0.2) (layer "B.Cu") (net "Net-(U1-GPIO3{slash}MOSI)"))
 (segment (start 208.28 90.17) (end 214.122 84.328) (width 0.2) (layer "B.Cu") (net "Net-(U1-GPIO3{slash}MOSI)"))
 (segment (start 162.455 88.414) (end 164.211 90.17) (width 0.2) (layer "B.Cu") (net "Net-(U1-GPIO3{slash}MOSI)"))
 (segment (start 162.455 86.4975) (end 162.455 88.414) (width 0.2) (layer "B.Cu") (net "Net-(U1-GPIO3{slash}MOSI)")))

